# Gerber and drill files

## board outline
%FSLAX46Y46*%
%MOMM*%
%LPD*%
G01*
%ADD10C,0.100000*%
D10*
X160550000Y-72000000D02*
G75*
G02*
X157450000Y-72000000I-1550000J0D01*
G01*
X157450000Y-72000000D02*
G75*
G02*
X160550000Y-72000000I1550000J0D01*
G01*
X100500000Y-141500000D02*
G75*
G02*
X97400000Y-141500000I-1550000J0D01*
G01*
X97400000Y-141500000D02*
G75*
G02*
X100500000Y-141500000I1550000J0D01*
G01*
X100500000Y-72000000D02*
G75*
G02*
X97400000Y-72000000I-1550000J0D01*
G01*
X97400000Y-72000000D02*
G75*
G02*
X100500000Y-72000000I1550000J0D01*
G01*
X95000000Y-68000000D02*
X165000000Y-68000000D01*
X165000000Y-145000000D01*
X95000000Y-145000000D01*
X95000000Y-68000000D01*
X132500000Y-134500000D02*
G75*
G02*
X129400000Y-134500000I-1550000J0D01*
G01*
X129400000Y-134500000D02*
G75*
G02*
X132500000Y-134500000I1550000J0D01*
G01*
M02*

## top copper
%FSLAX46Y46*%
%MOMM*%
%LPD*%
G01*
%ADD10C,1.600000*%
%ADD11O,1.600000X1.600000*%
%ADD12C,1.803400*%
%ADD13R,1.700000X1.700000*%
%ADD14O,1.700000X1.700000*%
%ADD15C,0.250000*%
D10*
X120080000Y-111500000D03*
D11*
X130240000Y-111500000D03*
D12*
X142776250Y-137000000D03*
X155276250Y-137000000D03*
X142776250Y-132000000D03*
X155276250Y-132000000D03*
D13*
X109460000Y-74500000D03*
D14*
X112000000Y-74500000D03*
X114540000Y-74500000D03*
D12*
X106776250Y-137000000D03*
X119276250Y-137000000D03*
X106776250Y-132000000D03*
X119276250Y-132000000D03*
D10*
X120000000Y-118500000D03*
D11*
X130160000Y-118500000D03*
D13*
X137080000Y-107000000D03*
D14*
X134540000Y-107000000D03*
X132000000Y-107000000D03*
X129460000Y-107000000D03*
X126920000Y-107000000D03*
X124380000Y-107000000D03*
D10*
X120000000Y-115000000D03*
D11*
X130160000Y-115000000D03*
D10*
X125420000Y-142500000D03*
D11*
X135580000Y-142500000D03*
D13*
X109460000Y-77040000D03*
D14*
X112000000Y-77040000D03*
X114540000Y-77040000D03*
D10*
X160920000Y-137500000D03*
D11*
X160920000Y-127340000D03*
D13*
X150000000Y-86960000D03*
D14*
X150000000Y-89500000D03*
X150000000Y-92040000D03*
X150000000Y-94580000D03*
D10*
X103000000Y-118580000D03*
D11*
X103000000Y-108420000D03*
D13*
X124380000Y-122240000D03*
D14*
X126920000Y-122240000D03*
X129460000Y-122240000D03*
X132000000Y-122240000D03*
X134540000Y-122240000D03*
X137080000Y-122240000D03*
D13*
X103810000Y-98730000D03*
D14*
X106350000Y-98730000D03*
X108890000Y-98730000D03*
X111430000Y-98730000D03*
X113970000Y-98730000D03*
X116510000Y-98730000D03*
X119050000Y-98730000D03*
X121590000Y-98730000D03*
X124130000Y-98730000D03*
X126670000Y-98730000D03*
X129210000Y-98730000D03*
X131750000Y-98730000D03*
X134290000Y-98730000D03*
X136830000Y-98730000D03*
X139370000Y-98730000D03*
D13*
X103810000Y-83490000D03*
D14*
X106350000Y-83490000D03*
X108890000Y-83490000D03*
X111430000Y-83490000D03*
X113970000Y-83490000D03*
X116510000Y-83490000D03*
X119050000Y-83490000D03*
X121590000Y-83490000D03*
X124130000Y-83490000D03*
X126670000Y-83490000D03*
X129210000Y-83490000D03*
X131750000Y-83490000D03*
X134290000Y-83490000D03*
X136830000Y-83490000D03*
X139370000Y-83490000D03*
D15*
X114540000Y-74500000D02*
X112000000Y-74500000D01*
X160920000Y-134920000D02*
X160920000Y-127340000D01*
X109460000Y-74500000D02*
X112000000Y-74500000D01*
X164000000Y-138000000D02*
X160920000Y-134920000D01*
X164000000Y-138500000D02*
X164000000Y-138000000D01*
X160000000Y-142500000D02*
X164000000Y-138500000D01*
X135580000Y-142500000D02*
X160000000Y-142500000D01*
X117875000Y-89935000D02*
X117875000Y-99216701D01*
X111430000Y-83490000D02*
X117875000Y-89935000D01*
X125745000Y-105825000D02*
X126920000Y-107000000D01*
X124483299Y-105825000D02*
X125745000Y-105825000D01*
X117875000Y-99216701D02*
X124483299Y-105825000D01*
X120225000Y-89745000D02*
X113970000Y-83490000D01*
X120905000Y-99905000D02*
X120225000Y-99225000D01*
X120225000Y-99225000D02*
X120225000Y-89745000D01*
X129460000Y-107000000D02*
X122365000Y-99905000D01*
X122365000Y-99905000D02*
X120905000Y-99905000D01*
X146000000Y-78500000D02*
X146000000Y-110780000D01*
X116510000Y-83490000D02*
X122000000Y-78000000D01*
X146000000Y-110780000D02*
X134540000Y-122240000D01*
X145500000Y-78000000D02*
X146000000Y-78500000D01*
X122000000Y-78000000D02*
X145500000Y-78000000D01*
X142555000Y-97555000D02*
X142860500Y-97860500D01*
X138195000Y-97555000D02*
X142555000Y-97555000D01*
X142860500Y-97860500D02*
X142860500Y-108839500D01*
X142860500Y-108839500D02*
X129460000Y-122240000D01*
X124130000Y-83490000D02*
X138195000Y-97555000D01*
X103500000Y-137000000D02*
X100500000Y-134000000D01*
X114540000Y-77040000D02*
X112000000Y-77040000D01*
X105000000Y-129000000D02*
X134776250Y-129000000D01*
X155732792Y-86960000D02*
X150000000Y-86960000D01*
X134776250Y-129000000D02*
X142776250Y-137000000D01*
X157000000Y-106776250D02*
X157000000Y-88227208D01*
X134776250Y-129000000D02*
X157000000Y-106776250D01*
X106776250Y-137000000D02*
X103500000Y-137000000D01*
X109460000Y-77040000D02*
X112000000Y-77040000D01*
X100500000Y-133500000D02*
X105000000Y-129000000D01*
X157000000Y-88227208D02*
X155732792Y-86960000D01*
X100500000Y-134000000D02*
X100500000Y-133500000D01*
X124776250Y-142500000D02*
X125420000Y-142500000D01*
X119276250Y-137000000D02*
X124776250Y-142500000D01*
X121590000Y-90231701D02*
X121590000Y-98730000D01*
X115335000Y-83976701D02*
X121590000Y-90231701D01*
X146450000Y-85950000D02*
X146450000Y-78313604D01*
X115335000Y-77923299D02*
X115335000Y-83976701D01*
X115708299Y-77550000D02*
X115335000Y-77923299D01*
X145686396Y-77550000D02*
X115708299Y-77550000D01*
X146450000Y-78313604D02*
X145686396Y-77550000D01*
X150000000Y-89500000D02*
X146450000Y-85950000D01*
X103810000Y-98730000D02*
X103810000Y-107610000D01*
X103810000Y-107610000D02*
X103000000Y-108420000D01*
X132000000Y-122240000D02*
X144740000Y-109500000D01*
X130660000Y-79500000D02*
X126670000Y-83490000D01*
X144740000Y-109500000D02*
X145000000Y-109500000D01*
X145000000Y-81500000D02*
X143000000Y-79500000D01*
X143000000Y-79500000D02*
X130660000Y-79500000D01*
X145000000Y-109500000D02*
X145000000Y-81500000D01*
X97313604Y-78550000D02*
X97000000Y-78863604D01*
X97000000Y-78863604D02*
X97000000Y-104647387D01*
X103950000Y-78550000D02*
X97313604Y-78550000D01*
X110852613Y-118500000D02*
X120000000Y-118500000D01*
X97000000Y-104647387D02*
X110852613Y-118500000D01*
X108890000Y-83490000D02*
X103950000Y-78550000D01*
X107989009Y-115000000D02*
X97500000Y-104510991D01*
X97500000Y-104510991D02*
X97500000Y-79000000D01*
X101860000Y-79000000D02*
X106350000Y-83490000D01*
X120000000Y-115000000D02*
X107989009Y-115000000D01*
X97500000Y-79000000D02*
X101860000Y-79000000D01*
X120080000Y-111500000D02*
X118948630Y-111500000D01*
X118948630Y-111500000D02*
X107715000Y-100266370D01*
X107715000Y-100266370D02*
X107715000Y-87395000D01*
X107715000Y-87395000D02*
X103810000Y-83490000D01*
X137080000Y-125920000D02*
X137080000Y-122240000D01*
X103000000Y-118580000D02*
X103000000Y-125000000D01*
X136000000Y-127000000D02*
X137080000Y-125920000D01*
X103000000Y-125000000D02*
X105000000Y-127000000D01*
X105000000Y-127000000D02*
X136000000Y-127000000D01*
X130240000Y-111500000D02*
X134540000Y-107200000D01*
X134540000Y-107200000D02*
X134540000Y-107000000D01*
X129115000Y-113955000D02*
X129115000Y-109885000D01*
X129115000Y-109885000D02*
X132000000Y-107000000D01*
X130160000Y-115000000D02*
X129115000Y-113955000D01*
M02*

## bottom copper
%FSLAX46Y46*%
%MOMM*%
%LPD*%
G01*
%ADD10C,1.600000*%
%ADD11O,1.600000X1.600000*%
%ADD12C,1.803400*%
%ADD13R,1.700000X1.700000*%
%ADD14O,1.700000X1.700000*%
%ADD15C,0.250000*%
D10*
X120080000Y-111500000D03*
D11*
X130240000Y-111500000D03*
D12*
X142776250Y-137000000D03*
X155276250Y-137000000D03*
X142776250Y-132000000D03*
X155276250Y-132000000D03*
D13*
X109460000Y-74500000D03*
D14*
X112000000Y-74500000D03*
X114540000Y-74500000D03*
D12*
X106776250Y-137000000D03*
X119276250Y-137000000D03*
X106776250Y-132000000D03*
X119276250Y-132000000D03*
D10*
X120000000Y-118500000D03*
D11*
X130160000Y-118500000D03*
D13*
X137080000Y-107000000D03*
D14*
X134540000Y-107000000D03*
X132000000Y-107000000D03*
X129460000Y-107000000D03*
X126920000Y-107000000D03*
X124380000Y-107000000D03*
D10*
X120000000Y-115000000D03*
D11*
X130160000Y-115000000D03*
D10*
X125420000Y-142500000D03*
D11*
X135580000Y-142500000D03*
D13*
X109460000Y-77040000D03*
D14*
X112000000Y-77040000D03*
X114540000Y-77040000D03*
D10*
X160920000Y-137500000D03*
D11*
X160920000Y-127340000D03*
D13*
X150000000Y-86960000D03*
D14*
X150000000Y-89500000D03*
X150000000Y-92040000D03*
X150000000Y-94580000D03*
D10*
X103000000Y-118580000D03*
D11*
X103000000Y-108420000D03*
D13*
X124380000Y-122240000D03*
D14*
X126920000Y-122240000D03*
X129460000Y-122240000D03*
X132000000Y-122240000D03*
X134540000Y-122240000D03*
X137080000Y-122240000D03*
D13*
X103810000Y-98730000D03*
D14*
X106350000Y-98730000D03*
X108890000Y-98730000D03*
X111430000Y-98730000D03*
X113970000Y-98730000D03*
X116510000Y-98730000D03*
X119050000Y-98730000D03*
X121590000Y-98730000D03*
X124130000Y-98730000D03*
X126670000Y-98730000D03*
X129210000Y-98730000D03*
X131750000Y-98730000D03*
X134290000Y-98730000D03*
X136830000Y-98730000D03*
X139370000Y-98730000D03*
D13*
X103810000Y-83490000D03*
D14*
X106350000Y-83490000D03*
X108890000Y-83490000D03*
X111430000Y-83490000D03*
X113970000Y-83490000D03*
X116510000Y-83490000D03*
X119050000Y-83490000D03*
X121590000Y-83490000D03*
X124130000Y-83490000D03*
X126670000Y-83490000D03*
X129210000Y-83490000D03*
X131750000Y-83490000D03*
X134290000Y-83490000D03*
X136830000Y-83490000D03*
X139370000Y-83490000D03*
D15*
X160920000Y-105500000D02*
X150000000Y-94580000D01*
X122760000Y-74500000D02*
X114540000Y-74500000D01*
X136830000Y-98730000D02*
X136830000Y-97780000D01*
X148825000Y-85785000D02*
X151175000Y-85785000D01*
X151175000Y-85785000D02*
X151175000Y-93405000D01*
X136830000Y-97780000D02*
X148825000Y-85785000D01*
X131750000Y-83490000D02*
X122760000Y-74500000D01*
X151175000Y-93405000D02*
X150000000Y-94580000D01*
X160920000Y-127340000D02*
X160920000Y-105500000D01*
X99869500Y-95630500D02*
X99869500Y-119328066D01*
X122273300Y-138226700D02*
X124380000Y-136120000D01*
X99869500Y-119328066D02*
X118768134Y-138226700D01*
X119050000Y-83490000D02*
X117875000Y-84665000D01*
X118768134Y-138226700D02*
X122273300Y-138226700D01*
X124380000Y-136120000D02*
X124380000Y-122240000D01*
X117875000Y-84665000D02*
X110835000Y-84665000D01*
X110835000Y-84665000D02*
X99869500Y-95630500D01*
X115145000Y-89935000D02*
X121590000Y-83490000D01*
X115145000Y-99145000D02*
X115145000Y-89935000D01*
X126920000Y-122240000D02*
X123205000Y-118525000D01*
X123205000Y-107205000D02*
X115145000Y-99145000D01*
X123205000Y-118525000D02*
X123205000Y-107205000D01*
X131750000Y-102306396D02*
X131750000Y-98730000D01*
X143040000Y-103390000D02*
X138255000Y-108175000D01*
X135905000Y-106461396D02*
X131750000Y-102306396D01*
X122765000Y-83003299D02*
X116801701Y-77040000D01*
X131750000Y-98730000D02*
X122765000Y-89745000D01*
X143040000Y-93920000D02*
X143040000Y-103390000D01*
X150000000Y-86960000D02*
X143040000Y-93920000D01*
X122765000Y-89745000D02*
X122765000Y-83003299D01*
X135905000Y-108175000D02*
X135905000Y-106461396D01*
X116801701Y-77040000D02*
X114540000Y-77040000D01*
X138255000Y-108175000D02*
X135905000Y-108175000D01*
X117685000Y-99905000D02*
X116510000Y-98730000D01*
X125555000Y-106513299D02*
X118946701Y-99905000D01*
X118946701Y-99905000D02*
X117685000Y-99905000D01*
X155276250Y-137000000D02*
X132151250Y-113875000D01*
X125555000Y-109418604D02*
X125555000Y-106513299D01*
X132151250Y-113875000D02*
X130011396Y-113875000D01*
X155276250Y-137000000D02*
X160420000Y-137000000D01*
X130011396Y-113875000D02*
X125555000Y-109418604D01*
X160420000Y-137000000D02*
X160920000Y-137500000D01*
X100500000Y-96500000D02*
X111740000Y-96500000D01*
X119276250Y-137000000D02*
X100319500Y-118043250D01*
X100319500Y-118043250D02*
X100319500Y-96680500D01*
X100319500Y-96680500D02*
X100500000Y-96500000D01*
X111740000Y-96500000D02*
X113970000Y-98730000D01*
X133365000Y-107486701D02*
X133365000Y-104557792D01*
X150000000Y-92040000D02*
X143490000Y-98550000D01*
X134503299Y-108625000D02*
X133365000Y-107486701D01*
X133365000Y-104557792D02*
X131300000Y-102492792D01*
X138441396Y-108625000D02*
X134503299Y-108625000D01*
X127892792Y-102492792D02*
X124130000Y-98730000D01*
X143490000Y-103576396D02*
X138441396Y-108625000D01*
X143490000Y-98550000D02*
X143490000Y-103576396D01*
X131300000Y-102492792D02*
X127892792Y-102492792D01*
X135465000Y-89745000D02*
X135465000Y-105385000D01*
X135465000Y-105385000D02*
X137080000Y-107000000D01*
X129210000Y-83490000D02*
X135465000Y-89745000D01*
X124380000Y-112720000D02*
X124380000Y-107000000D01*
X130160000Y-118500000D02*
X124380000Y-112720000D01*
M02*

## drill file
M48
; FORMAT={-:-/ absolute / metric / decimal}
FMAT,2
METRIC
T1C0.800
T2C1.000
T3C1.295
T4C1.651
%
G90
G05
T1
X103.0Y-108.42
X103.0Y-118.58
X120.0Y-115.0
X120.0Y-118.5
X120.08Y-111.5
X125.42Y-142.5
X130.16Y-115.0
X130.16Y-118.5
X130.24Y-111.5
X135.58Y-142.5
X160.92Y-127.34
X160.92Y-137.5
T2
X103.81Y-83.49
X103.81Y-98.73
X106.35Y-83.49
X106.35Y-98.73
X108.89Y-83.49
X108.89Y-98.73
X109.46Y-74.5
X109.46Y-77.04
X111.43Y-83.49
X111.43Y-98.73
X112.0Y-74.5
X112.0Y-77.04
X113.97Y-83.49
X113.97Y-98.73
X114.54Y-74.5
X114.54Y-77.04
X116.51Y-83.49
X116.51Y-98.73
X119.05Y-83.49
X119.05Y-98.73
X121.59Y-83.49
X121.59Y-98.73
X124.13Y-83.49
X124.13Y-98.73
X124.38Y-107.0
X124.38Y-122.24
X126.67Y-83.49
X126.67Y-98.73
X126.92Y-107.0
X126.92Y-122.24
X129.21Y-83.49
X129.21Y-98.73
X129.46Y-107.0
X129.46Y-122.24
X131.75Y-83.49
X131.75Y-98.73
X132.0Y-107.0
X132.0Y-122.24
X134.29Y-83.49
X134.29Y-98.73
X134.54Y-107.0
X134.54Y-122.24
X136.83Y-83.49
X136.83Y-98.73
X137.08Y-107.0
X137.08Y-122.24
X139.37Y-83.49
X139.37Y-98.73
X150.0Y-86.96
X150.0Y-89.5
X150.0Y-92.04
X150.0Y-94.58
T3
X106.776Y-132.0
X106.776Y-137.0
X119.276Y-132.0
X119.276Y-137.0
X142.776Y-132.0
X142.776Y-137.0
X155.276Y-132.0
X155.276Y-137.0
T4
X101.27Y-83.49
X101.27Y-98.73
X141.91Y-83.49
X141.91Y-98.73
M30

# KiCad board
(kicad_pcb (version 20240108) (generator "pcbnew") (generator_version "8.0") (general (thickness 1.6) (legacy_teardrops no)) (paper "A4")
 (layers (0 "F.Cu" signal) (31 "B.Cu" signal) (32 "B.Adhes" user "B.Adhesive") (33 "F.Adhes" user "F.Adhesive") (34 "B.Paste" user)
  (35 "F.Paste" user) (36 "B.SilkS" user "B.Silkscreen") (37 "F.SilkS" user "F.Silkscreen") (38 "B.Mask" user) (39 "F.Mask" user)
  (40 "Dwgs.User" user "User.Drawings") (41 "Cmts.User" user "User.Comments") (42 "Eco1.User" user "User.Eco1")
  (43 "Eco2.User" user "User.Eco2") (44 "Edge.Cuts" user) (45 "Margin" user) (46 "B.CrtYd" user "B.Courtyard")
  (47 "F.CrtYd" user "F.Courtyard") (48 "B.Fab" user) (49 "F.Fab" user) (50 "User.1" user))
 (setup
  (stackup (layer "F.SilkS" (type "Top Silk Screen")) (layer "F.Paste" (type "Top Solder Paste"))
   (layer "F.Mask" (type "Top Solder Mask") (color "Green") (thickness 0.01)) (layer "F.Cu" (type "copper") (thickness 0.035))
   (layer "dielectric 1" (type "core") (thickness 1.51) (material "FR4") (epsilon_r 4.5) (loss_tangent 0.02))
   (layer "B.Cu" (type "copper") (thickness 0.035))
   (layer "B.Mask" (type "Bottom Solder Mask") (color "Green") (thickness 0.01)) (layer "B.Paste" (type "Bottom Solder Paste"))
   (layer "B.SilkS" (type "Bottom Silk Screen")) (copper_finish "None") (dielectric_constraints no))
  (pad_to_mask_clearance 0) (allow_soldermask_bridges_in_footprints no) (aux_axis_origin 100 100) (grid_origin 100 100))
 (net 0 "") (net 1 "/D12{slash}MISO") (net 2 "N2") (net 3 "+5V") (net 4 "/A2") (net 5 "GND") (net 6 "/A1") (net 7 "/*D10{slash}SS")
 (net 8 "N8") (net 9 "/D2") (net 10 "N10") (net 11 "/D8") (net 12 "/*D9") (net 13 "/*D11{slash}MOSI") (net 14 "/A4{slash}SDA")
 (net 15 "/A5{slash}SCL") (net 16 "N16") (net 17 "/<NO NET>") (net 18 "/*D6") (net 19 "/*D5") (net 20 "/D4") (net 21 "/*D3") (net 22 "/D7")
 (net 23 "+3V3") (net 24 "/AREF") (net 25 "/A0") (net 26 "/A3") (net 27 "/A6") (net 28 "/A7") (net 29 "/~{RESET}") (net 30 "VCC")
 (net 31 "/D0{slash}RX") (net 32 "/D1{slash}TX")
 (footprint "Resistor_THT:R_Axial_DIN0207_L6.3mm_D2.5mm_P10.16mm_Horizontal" (layer "F.Cu") (at 120.08 111.5)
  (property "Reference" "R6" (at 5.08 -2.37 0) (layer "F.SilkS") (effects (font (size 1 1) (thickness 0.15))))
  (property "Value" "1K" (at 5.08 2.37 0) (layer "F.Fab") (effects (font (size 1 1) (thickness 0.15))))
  (pad "1" thru_hole circle (at 0 0) (size 1.6 1.6) (drill 0.8) (layers "*.Cu" "*.Mask") (remove_unused_layers no) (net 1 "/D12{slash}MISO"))
  (pad "2" thru_hole oval (at 10.16 0) (size 1.6 1.6) (drill 0.8) (layers "*.Cu" "*.Mask") (remove_unused_layers no) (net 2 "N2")))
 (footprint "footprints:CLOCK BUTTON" (layer "F.Cu") (at 142.77625 137)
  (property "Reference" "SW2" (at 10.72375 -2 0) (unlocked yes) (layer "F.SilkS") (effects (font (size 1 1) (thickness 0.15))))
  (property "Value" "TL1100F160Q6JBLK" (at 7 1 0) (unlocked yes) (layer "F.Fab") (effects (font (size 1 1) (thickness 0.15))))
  (pad "1" thru_hole circle (at 0 0) (size 1.8034 1.8034) (drill 1.2954) (layers "*.Cu" "*.Mask") (remove_unused_layers no) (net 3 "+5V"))
  (pad "2" thru_hole circle (at 12.5 0) (size 1.8034 1.8034) (drill 1.2954) (layers "*.Cu" "*.Mask") (remove_unused_layers no) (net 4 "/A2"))
  (pad "3" thru_hole circle (at 0 -5) (size 1.8034 1.8034) (drill 1.2954) (layers "*.Cu" "*.Mask") (remove_unused_layers no))
  (pad "4" thru_hole circle (at 12.5 -5) (size 1.8034 1.8034) (drill 1.2954) (layers "*.Cu" "*.Mask") (remove_unused_layers no)))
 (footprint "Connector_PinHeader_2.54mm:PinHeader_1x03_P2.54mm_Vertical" (layer "F.Cu") (at 109.46 74.5 90)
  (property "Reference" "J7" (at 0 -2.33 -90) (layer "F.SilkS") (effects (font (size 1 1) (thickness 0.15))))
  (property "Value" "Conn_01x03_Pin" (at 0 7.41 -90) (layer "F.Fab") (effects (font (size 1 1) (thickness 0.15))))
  (pad "1" thru_hole rect (at 0 0 90) (size 1.7 1.7) (drill 1) (layers "*.Cu" "*.Mask") (remove_unused_layers no) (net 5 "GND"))
  (pad "2" thru_hole oval (at 0 2.54 90) (size 1.7 1.7) (drill 1) (layers "*.Cu" "*.Mask") (remove_unused_layers no) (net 5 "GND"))
  (pad "3" thru_hole oval (at 0 5.08 90) (size 1.7 1.7) (drill 1) (layers "*.Cu" "*.Mask") (remove_unused_layers no) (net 5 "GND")))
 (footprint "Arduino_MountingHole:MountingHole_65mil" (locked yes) (layer "F.Cu") (at 101.27 83.49)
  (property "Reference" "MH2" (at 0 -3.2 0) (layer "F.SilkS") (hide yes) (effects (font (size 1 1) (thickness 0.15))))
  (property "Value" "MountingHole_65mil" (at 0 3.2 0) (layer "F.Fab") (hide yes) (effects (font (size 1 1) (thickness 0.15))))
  (pad "" np_thru_hole circle (at 0 0) (size 1.651 1.651) (drill 1.651) (layers "F&B.Cu" "*.Mask")))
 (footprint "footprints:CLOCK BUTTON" (layer "F.Cu") (at 106.77625 137)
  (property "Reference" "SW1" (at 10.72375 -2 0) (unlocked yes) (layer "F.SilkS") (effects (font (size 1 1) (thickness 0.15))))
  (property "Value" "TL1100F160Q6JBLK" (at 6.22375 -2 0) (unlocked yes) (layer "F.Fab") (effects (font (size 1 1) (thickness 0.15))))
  (pad "1" thru_hole circle (at 0 0) (size 1.8034 1.8034) (drill 1.2954) (layers "*.Cu" "*.Mask") (remove_unused_layers no) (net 3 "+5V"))
  (pad "2" thru_hole circle (at 12.5 0) (size 1.8034 1.8034) (drill 1.2954) (layers "*.Cu" "*.Mask") (remove_unused_layers no) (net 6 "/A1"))
  (pad "3" thru_hole circle (at 0 -5) (size 1.8034 1.8034) (drill 1.2954) (layers "*.Cu" "*.Mask") (remove_unused_layers no))
  (pad "4" thru_hole circle (at 12.5 -5) (size 1.8034 1.8034) (drill 1.2954) (layers "*.Cu" "*.Mask") (remove_unused_layers no)))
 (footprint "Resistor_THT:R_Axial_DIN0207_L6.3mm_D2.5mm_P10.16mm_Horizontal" (layer "F.Cu") (at 120 118.5)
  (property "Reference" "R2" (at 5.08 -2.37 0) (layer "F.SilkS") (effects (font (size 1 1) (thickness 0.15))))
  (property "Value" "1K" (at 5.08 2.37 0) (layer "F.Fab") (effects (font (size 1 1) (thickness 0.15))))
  (pad "1" thru_hole circle (at 0 0) (size 1.6 1.6) (drill 0.8) (layers "*.Cu" "*.Mask") (remove_unused_layers no) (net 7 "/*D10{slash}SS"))
  (pad "2" thru_hole oval (at 10.16 0) (size 1.6 1.6) (drill 0.8) (layers "*.Cu" "*.Mask") (remove_unused_layers no) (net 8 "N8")))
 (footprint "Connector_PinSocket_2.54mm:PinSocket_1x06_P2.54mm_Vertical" (layer "F.Cu") (at 137.08 107 -90)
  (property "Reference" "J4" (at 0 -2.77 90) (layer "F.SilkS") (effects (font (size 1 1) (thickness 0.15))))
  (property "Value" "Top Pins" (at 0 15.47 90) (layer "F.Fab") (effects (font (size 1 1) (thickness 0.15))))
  (pad "1" thru_hole rect (at 0 0 270) (size 1.7 1.7) (drill 1) (layers "*.Cu" "*.Mask") (remove_unused_layers no) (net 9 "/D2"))
  (pad "2" thru_hole oval (at 0 2.54 270) (size 1.7 1.7) (drill 1) (layers "*.Cu" "*.Mask") (remove_unused_layers no) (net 2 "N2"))
  (pad "3" thru_hole oval (at 0 5.08 270) (size 1.7 1.7) (drill 1) (layers "*.Cu" "*.Mask") (remove_unused_layers no) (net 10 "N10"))
  (pad "4" thru_hole oval (at 0 7.62 270) (size 1.7 1.7) (drill 1) (layers "*.Cu" "*.Mask") (remove_unused_layers no) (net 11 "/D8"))
  (pad "5" thru_hole oval (at 0 10.16 270) (size 1.7 1.7) (drill 1) (layers "*.Cu" "*.Mask") (remove_unused_layers no) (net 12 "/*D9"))
  (pad "6" thru_hole oval (at 0 12.7 270) (size 1.7 1.7) (drill 1) (layers "*.Cu" "*.Mask") (remove_unused_layers no) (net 8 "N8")))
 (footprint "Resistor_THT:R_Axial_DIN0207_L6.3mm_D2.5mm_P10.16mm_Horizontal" (layer "F.Cu") (at 120 115)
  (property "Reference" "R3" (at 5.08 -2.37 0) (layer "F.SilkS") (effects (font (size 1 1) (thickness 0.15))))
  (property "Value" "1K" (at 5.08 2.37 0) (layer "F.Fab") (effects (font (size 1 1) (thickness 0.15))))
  (pad "1" thru_hole circle (at 0 0) (size 1.6 1.6) (drill 0.8) (layers "*.Cu" "*.Mask") (remove_unused_layers no)
   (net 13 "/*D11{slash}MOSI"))
  (pad "2" thru_hole oval (at 10.16 0) (size 1.6 1.6) (drill 0.8) (layers "*.Cu" "*.Mask") (remove_unused_layers no) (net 10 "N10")))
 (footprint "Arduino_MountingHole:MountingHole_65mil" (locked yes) (layer "F.Cu") (at 141.91 98.73)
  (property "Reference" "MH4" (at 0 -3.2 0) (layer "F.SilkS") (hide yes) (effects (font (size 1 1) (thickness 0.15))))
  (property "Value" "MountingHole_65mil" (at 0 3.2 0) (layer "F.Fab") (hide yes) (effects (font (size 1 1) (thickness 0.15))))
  (pad "" np_thru_hole circle (at 0 0) (size 1.651 1.651) (drill 1.651) (layers "F&B.Cu" "*.Mask")))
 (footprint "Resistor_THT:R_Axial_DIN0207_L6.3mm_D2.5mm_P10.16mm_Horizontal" (layer "F.Cu") (at 125.42 142.5)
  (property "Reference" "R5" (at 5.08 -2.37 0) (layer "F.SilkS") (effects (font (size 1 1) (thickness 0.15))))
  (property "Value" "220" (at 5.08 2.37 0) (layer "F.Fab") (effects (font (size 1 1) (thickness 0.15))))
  (pad "1" thru_hole circle (at 0 0) (size 1.6 1.6) (drill 0.8) (layers "*.Cu" "*.Mask") (remove_unused_layers no) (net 6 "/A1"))
  (pad "2" thru_hole oval (at 10.16 0) (size 1.6 1.6) (drill 0.8) (layers "*.Cu" "*.Mask") (remove_unused_layers no) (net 5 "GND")))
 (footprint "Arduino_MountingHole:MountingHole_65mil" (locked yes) (layer "F.Cu") (at 101.27 98.73)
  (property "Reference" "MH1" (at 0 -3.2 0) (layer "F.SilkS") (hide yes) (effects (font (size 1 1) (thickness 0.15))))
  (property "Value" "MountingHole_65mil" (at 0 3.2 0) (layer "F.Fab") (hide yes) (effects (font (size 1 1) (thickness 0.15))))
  (pad "" np_thru_hole circle (at 0 0) (size 1.651 1.651) (drill 1.651) (layers "F&B.Cu" "*.Mask")))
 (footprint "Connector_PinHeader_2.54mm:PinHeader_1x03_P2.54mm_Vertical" (layer "F.Cu") (at 109.46 77.04 90)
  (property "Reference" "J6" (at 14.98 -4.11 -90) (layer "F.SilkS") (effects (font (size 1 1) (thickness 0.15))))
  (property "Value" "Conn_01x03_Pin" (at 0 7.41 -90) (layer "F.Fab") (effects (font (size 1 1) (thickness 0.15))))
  (pad "1" thru_hole rect (at 0 0 90) (size 1.7 1.7) (drill 1) (layers "*.Cu" "*.Mask") (remove_unused_layers no) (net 3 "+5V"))
  (pad "2" thru_hole oval (at 0 2.54 90) (size 1.7 1.7) (drill 1) (layers "*.Cu" "*.Mask") (remove_unused_layers no) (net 3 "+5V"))
  (pad "3" thru_hole oval (at 0 5.08 90) (size 1.7 1.7) (drill 1) (layers "*.Cu" "*.Mask") (remove_unused_layers no) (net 3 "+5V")))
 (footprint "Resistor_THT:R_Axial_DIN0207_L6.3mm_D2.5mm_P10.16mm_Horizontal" (layer "F.Cu") (at 160.92 137.5 90)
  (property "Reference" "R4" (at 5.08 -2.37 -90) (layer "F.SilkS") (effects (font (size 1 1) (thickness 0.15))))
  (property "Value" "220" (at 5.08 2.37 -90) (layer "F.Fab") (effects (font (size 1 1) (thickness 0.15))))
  (pad "1" thru_hole circle (at 0 0 90) (size 1.6 1.6) (drill 0.8) (layers "*.Cu" "*.Mask") (remove_unused_layers no) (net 4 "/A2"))
  (pad "2" thru_hole oval (at 10.16 0 90) (size 1.6 1.6) (drill 0.8) (layers "*.Cu" "*.Mask") (remove_unused_layers no) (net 5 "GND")))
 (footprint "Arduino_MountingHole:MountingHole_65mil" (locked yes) (layer "F.Cu") (at 141.91 83.49)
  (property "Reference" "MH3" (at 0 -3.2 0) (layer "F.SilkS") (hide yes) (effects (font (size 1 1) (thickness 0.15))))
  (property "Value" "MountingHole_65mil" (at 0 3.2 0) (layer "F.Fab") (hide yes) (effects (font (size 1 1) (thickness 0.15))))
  (pad "" np_thru_hole circle (at 0 0) (size 1.651 1.651) (drill 1.651) (layers "F&B.Cu" "*.Mask")))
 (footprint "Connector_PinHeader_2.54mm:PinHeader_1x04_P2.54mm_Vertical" (layer "F.Cu") (at 150 86.96)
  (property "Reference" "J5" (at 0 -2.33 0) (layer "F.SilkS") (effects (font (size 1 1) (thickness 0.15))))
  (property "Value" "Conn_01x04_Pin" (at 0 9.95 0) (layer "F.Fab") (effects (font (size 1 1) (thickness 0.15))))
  (pad "1" thru_hole rect (at 0 0) (size 1.7 1.7) (drill 1) (layers "*.Cu" "*.Mask") (remove_unused_layers no) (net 3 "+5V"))
  (pad "2" thru_hole oval (at 0 2.54) (size 1.7 1.7) (drill 1) (layers "*.Cu" "*.Mask") (remove_unused_layers no) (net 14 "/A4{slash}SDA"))
  (pad "3" thru_hole oval (at 0 5.08) (size 1.7 1.7) (drill 1) (layers "*.Cu" "*.Mask") (remove_unused_layers no) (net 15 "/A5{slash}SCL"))
  (pad "4" thru_hole oval (at 0 7.62) (size 1.7 1.7) (drill 1) (layers "*.Cu" "*.Mask") (remove_unused_layers no) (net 5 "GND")))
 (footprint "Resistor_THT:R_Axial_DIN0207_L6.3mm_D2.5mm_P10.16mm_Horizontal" (layer "F.Cu") (at 103 118.58 90)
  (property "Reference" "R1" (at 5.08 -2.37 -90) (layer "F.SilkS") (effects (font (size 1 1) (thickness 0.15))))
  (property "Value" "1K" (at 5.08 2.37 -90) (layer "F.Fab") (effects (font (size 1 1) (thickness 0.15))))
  (pad "1" thru_hole circle (at 0 0 90) (size 1.6 1.6) (drill 0.8) (layers "*.Cu" "*.Mask") (remove_unused_layers no) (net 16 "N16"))
  (pad "2" thru_hole oval (at 10.16 0 90) (size 1.6 1.6) (drill 0.8) (layers "*.Cu" "*.Mask") (remove_unused_layers no) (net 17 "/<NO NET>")))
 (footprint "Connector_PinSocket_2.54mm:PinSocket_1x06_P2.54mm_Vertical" (layer "F.Cu") (at 124.38 122.24 90)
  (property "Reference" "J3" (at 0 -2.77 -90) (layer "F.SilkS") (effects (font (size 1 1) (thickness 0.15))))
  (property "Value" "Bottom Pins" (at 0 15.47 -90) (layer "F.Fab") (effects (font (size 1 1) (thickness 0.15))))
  (pad "1" thru_hole rect (at 0 0 90) (size 1.7 1.7) (drill 1) (layers "*.Cu" "*.Mask") (remove_unused_layers no) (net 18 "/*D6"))
  (pad "2" thru_hole oval (at 0 2.54 90) (size 1.7 1.7) (drill 1) (layers "*.Cu" "*.Mask") (remove_unused_layers no) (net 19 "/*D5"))
  (pad "3" thru_hole oval (at 0 5.08 90) (size 1.7 1.7) (drill 1) (layers "*.Cu" "*.Mask") (remove_unused_layers no) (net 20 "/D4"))
  (pad "4" thru_hole oval (at 0 7.62 90) (size 1.7 1.7) (drill 1) (layers "*.Cu" "*.Mask") (remove_unused_layers no) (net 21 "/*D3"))
  (pad "5" thru_hole oval (at 0 10.16 90) (size 1.7 1.7) (drill 1) (layers "*.Cu" "*.Mask") (remove_unused_layers no) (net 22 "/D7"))
  (pad "6" thru_hole oval (at 0 12.7 90) (size 1.7 1.7) (drill 1) (layers "*.Cu" "*.Mask") (remove_unused_layers no) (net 16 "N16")))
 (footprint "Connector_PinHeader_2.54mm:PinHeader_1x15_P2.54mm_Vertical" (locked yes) (layer "B.Cu") (at 103.81 98.73 -90)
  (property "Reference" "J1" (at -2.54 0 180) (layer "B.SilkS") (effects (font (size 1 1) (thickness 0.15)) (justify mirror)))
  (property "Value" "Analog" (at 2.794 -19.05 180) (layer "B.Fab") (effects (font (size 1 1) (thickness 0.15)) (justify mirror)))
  (pad "1" thru_hole rect (at 0 0 270) (size 1.7 1.7) (drill 1) (layers "*.Cu" "*.Mask") (remove_unused_layers no) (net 17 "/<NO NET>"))
  (pad "2" thru_hole oval (at 0 -2.54 270) (size 1.7 1.7) (drill 1) (layers "*.Cu" "*.Mask") (remove_unused_layers no) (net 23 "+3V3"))
  (pad "3" thru_hole oval (at 0 -5.08 270) (size 1.7 1.7) (drill 1) (layers "*.Cu" "*.Mask") (remove_unused_layers no) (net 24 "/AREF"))
  (pad "4" thru_hole oval (at 0 -7.62 270) (size 1.7 1.7) (drill 1) (layers "*.Cu" "*.Mask") (remove_unused_layers no) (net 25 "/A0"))
  (pad "5" thru_hole oval (at 0 -10.16 270) (size 1.7 1.7) (drill 1) (layers "*.Cu" "*.Mask") (remove_unused_layers no) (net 6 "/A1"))
  (pad "6" thru_hole oval (at 0 -12.7 270) (size 1.7 1.7) (drill 1) (layers "*.Cu" "*.Mask") (remove_unused_layers no) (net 4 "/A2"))
  (pad "7" thru_hole oval (at 0 -15.24 270) (size 1.7 1.7) (drill 1) (layers "*.Cu" "*.Mask") (remove_unused_layers no) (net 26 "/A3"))
  (pad "8" thru_hole oval (at 0 -17.78 270) (size 1.7 1.7) (drill 1) (layers "*.Cu" "*.Mask") (remove_unused_layers no)
   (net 14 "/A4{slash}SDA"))
  (pad "9" thru_hole oval (at 0 -20.32 270) (size 1.7 1.7) (drill 1) (layers "*.Cu" "*.Mask") (remove_unused_layers no)
   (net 15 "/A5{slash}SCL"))
  (pad "10" thru_hole oval (at 0 -22.86 270) (size 1.7 1.7) (drill 1) (layers "*.Cu" "*.Mask") (remove_unused_layers no) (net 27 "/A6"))
  (pad "11" thru_hole oval (at 0 -25.4 270) (size 1.7 1.7) (drill 1) (layers "*.Cu" "*.Mask") (remove_unused_layers no) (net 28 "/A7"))
  (pad "12" thru_hole oval (at 0 -27.94 270) (size 1.7 1.7) (drill 1) (layers "*.Cu" "*.Mask") (remove_unused_layers no) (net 3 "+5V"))
  (pad "13" thru_hole oval (at 0 -30.48 270) (size 1.7 1.7) (drill 1) (layers "*.Cu" "*.Mask") (remove_unused_layers no)
   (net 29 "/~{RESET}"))
  (pad "14" thru_hole oval (at 0 -33.02 270) (size 1.7 1.7) (drill 1) (layers "*.Cu" "*.Mask") (remove_unused_layers no) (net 5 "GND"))
  (pad "15" thru_hole oval (at 0 -35.56 270) (size 1.7 1.7) (drill 1) (layers "*.Cu" "*.Mask") (remove_unused_layers no) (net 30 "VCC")))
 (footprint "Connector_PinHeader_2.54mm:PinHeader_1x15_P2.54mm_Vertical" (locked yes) (layer "B.Cu") (at 103.81 83.49 -90)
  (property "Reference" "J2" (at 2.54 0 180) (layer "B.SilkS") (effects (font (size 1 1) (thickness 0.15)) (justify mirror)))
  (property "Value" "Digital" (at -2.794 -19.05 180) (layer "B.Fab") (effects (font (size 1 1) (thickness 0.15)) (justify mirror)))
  (pad "1" thru_hole rect (at 0 0 270) (size 1.7 1.7) (drill 1) (layers "*.Cu" "*.Mask") (remove_unused_layers no) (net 1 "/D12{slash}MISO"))
  (pad "2" thru_hole oval (at 0 -2.54 270) (size 1.7 1.7) (drill 1) (layers "*.Cu" "*.Mask") (remove_unused_layers no)
   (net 13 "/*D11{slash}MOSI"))
  (pad "3" thru_hole oval (at 0 -5.08 270) (size 1.7 1.7) (drill 1) (layers "*.Cu" "*.Mask") (remove_unused_layers no)
   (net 7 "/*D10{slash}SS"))
  (pad "4" thru_hole oval (at 0 -7.62 270) (size 1.7 1.7) (drill 1) (layers "*.Cu" "*.Mask") (remove_unused_layers no) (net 12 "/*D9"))
  (pad "5" thru_hole oval (at 0 -10.16 270) (size 1.7 1.7) (drill 1) (layers "*.Cu" "*.Mask") (remove_unused_layers no) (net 11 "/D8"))
  (pad "6" thru_hole oval (at 0 -12.7 270) (size 1.7 1.7) (drill 1) (layers "*.Cu" "*.Mask") (remove_unused_layers no) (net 22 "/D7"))
  (pad "7" thru_hole oval (at 0 -15.24 270) (size 1.7 1.7) (drill 1) (layers "*.Cu" "*.Mask") (remove_unused_layers no) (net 18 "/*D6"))
  (pad "8" thru_hole oval (at 0 -17.78 270) (size 1.7 1.7) (drill 1) (layers "*.Cu" "*.Mask") (remove_unused_layers no) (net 19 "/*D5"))
  (pad "9" thru_hole oval (at 0 -20.32 270) (size 1.7 1.7) (drill 1) (layers "*.Cu" "*.Mask") (remove_unused_layers no) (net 20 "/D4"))
  (pad "10" thru_hole oval (at 0 -22.86 270) (size 1.7 1.7) (drill 1) (layers "*.Cu" "*.Mask") (remove_unused_layers no) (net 21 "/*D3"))
  (pad "11" thru_hole oval (at 0 -25.4 270) (size 1.7 1.7) (drill 1) (layers "*.Cu" "*.Mask") (remove_unused_layers no) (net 9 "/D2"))
  (pad "12" thru_hole oval (at 0 -27.94 270) (size 1.7 1.7) (drill 1) (layers "*.Cu" "*.Mask") (remove_unused_layers no) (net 5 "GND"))
  (pad "13" thru_hole oval (at 0 -30.48 270) (size 1.7 1.7) (drill 1) (layers "*.Cu" "*.Mask") (remove_unused_layers no)
   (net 29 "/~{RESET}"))
  (pad "14" thru_hole oval (at 0 -33.02 270) (size 1.7 1.7) (drill 1) (layers "*.Cu" "*.Mask") (remove_unused_layers no)
   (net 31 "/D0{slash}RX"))
  (pad "15" thru_hole oval (at 0 -35.56 270) (size 1.7 1.7) (drill 1) (layers "*.Cu" "*.Mask") (remove_unused_layers no)
   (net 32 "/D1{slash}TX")))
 (gr_circle (center 159 72) (end 160.55 72) (stroke (width 0.1) (type default)) (fill none) (layer "Edge.Cuts"))
 (gr_circle (center 98.95 141.5) (end 100.5 141.5) (stroke (width 0.1) (type default)) (fill none) (layer "Edge.Cuts"))
 (gr_circle (center 98.95 72) (end 100.5 72) (stroke (width 0.1) (type default)) (fill none) (layer "Edge.Cuts"))
 (gr_rect (start 95 68) (end 165 145) (stroke (width 0.1) (type default)) (fill none) (layer "Edge.Cuts"))
 (gr_circle (center 130.95 134.5) (end 132.5 134.5) (stroke (width 0.1) (type default)) (fill none) (layer "Edge.Cuts"))
 (segment (start 114.54 74.5) (end 112 74.5) (width 0.25) (layer "F.Cu") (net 5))
 (segment (start 160.92 134.92) (end 160.92 127.34) (width 0.25) (layer "F.Cu") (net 5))
 (segment (start 109.46 74.5) (end 112 74.5) (width 0.25) (layer "F.Cu") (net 5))
 (segment (start 164 138) (end 160.92 134.92) (width 0.25) (layer "F.Cu") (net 5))
 (segment (start 164 138.5) (end 164 138) (width 0.25) (layer "F.Cu") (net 5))
 (segment (start 160 142.5) (end 164 138.5) (width 0.25) (layer "F.Cu") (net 5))
 (segment (start 135.58 142.5) (end 160 142.5) (width 0.25) (layer "F.Cu") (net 5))
 (segment (start 160.92 105.5) (end 150 94.58) (width 0.25) (layer "B.Cu") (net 5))
 (segment (start 122.76 74.5) (end 114.54 74.5) (width 0.25) (layer "B.Cu") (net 5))
 (segment (start 136.83 98.73) (end 136.83 97.78) (width 0.25) (layer "B.Cu") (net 5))
 (segment (start 148.825 85.785) (end 151.175 85.785) (width 0.25) (layer "B.Cu") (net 5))
 (segment (start 151.175 85.785) (end 151.175 93.405) (width 0.25) (layer "B.Cu") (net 5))
 (segment (start 136.83 97.78) (end 148.825 85.785) (width 0.25) (layer "B.Cu") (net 5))
 (segment (start 131.75 83.49) (end 122.76 74.5) (width 0.25) (layer "B.Cu") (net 5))
 (segment (start 151.175 93.405) (end 150 94.58) (width 0.25) (layer "B.Cu") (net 5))
 (segment (start 160.92 127.34) (end 160.92 105.5) (width 0.25) (layer "B.Cu") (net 5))
 (segment (start 117.875 89.935) (end 117.875 99.216701) (width 0.25) (layer "F.Cu") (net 12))
 (segment (start 111.43 83.49) (end 117.875 89.935) (width 0.25) (layer "F.Cu") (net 12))
 (segment (start 125.745 105.825) (end 126.92 107) (width 0.25) (layer "F.Cu") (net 12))
 (segment (start 124.483299 105.825) (end 125.745 105.825) (width 0.25) (layer "F.Cu") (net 12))
 (segment (start 117.875 99.216701) (end 124.483299 105.825) (width 0.25) (layer "F.Cu") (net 12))
 (segment (start 120.225 89.745) (end 113.97 83.49) (width 0.25) (layer "F.Cu") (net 11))
 (segment (start 120.905 99.905) (end 120.225 99.225) (width 0.25) (layer "F.Cu") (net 11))
 (segment (start 120.225 99.225) (end 120.225 89.745) (width 0.25) (layer "F.Cu") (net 11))
 (segment (start 129.46 107) (end 122.365 99.905) (width 0.25) (layer "F.Cu") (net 11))
 (segment (start 122.365 99.905) (end 120.905 99.905) (width 0.25) (layer "F.Cu") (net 11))
 (segment (start 146 78.5) (end 146 110.78) (width 0.25) (layer "F.Cu") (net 22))
 (segment (start 116.51 83.49) (end 122 78) (width 0.25) (layer "F.Cu") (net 22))
 (segment (start 146 110.78) (end 134.54 122.24) (width 0.25) (layer "F.Cu") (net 22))
 (segment (start 145.5 78) (end 146 78.5) (width 0.25) (layer "F.Cu") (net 22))
 (segment (start 122 78) (end 145.5 78) (width 0.25) (layer "F.Cu") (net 22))
 (segment (start 99.8695 95.6305) (end 99.8695 119.328066) (width 0.25) (layer "B.Cu") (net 18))
 (segment (start 122.2733 138.2267) (end 124.38 136.12) (width 0.25) (layer "B.Cu") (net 18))
 (segment (start 99.8695 119.328066) (end 118.768134 138.2267) (width 0.25) (layer "B.Cu") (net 18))
 (segment (start 119.05 83.49) (end 117.875 84.665) (width 0.25) (layer "B.Cu") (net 18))
 (segment (start 118.768134 138.2267) (end 122.2733 138.2267) (width 0.25) (layer "B.Cu") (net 18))
 (segment (start 124.38 136.12) (end 124.38 122.24) (width 0.25) (layer "B.Cu") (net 18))
 (segment (start 117.875 84.665) (end 110.835 84.665) (width 0.25) (layer "B.Cu") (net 18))
 (segment (start 110.835 84.665) (end 99.8695 95.6305) (width 0.25) (layer "B.Cu") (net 18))
 (segment (start 115.145 89.935) (end 121.59 83.49) (width 0.25) (layer "B.Cu") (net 19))
 (segment (start 115.145 99.145) (end 115.145 89.935) (width 0.25) (layer "B.Cu") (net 19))
 (segment (start 126.92 122.24) (end 123.205 118.525) (width 0.25) (layer "B.Cu") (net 19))
 (segment (start 123.205 107.205) (end 115.145 99.145) (width 0.25) (layer "B.Cu") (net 19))
 (segment (start 123.205 118.525) (end 123.205 107.205) (width 0.25) (layer "B.Cu") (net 19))
 (segment (start 142.555 97.555) (end 142.8605 97.8605) (width 0.25) (layer "F.Cu") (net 20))
 (segment (start 138.195 97.555) (end 142.555 97.555) (width 0.25) (layer "F.Cu") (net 20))
 (segment (start 142.8605 97.8605) (end 142.8605 108.8395) (width 0.25) (layer "F.Cu") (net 20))
 (segment (start 142.8605 108.8395) (end 129.46 122.24) (width 0.25) (layer "F.Cu") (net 20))
 (segment (start 124.13 83.49) (end 138.195 97.555) (width 0.25) (layer "F.Cu") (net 20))
 (segment (start 103.5 137) (end 100.5 134) (width 0.25) (layer "F.Cu") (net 3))
 (segment (start 114.54 77.04) (end 112 77.04) (width 0.25) (layer "F.Cu") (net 3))
 (segment (start 105 129) (end 134.77625 129) (width 0.25) (layer "F.Cu") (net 3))
 (segment (start 155.732792 86.96) (end 150 86.96) (width 0.25) (layer "F.Cu") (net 3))
 (segment (start 134.77625 129) (end 142.77625 137) (width 0.25) (layer "F.Cu") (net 3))
 (segment (start 157 106.77625) (end 157 88.227208) (width 0.25) (layer "F.Cu") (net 3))
 (segment (start 134.77625 129) (end 157 106.77625) (width 0.25) (layer "F.Cu") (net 3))
 (segment (start 106.77625 137) (end 103.5 137) (width 0.25) (layer "F.Cu") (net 3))
 (segment (start 109.46 77.04) (end 112 77.04) (width 0.25) (layer "F.Cu") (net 3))
 (segment (start 100.5 133.5) (end 105 129) (width 0.25) (layer "F.Cu") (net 3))
 (segment (start 157 88.227208) (end 155.732792 86.96) (width 0.25) (layer "F.Cu") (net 3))
 (segment (start 100.5 134) (end 100.5 133.5) (width 0.25) (layer "F.Cu") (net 3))
 (segment (start 131.75 102.306396) (end 131.75 98.73) (width 0.25) (layer "B.Cu") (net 3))
 (segment (start 143.04 103.39) (end 138.255 108.175) (width 0.25) (layer "B.Cu") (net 3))
 (segment (start 135.905 106.461396) (end 131.75 102.306396) (width 0.25) (layer "B.Cu") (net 3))
 (segment (start 122.765 83.003299) (end 116.801701 77.04) (width 0.25) (layer "B.Cu") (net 3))
 (segment (start 131.75 98.73) (end 122.765 89.745) (width 0.25) (layer "B.Cu") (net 3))
 (segment (start 143.04 93.92) (end 143.04 103.39) (width 0.25) (layer "B.Cu") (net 3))
 (segment (start 150 86.96) (end 143.04 93.92) (width 0.25) (layer "B.Cu") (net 3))
 (segment (start 122.765 89.745) (end 122.765 83.003299) (width 0.25) (layer "B.Cu") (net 3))
 (segment (start 135.905 108.175) (end 135.905 106.461396) (width 0.25) (layer "B.Cu") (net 3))
 (segment (start 116.801701 77.04) (end 114.54 77.04) (width 0.25) (layer "B.Cu") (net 3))
 (segment (start 138.255 108.175) (end 135.905 108.175) (width 0.25) (layer "B.Cu") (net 3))
 (segment (start 117.685 99.905) (end 116.51 98.73) (width 0.25) (layer "B.Cu") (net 4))
 (segment (start 125.555 106.513299) (end 118.946701 99.905) (width 0.25) (layer "B.Cu") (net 4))
 (segment (start 118.946701 99.905) (end 117.685 99.905) (width 0.25) (layer "B.Cu") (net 4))
 (segment (start 155.27625 137) (end 132.15125 113.875) (width 0.25) (layer "B.Cu") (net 4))
 (segment (start 125.555 109.418604) (end 125.555 106.513299) (width 0.25) (layer "B.Cu") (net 4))
 (segment (start 132.15125 113.875) (end 130.011396 113.875) (width 0.25) (layer "B.Cu") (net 4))
 (segment (start 155.27625 137) (end 160.42 137) (width 0.25) (layer "B.Cu") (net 4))
 (segment (start 130.011396 113.875) (end 125.555 109.418604) (width 0.25) (layer "B.Cu") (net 4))
 (segment (start 160.42 137) (end 160.92 137.5) (width 0.25) (layer "B.Cu") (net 4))
 (segment (start 124.77625 142.5) (end 125.42 142.5) (width 0.25) (layer "F.Cu") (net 6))
 (segment (start 119.27625 137) (end 124.77625 142.5) (width 0.25) (layer "F.Cu") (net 6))
 (segment (start 100.5 96.5) (end 111.74 96.5) (width 0.25) (layer "B.Cu") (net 6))
 (segment (start 119.27625 137) (end 100.3195 118.04325) (width 0.25) (layer "B.Cu") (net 6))
 (segment (start 100.3195 118.04325) (end 100.3195 96.6805) (width 0.25) (layer "B.Cu") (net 6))
 (segment (start 100.3195 96.6805) (end 100.5 96.5) (width 0.25) (layer "B.Cu") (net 6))
 (segment (start 111.74 96.5) (end 113.97 98.73) (width 0.25) (layer "B.Cu") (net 6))
 (segment (start 133.365 107.486701) (end 133.365 104.557792) (width 0.25) (layer "B.Cu") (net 15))
 (segment (start 150 92.04) (end 143.49 98.55) (width 0.25) (layer "B.Cu") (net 15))
 (segment (start 134.503299 108.625) (end 133.365 107.486701) (width 0.25) (layer "B.Cu") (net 15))
 (segment (start 133.365 104.557792) (end 131.3 102.492792) (width 0.25) (layer "B.Cu") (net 15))
 (segment (start 138.441396 108.625) (end 134.503299 108.625) (width 0.25) (layer "B.Cu") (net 15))
 (segment (start 127.892792 102.492792) (end 124.13 98.73) (width 0.25) (layer "B.Cu") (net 15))
 (segment (start 143.49 103.576396) (end 138.441396 108.625) (width 0.25) (layer "B.Cu") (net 15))
 (segment (start 143.49 98.55) (end 143.49 103.576396) (width 0.25) (layer "B.Cu") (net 15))
 (segment (start 131.3 102.492792) (end 127.892792 102.492792) (width 0.25) (layer "B.Cu") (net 15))
 (segment (start 121.59 90.231701) (end 121.59 98.73) (width 0.25) (layer "F.Cu") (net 14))
 (segment (start 115.335 83.976701) (end 121.59 90.231701) (width 0.25) (layer "F.Cu") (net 14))
 (segment (start 146.45 85.95) (end 146.45 78.313604) (width 0.25) (layer "F.Cu") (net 14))
 (segment (start 115.335 77.923299) (end 115.335 83.976701) (width 0.25) (layer "F.Cu") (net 14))
 (segment (start 115.708299 77.55) (end 115.335 77.923299) (width 0.25) (layer "F.Cu") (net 14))
 (segment (start 145.686396 77.55) (end 115.708299 77.55) (width 0.25) (layer "F.Cu") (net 14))
 (segment (start 146.45 78.313604) (end 145.686396 77.55) (width 0.25) (layer "F.Cu") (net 14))
 (segment (start 150 89.5) (end 146.45 85.95) (width 0.25) (layer "F.Cu") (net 14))
 (segment (start 103.81 98.73) (end 103.81 107.61) (width 0.25) (layer "F.Cu") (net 17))
 (segment (start 103.81 107.61) (end 103 108.42) (width 0.25) (layer "F.Cu") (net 17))
 (segment (start 135.465 89.745) (end 135.465 105.385) (width 0.25) (layer "B.Cu") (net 9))
 (segment (start 135.465 105.385) (end 137.08 107) (width 0.25) (layer "B.Cu") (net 9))
 (segment (start 129.21 83.49) (end 135.465 89.745) (width 0.25) (layer "B.Cu") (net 9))
 (segment (start 132 122.24) (end 144.74 109.5) (width 0.25) (layer "F.Cu") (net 21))
 (segment (start 130.66 79.5) (end 126.67 83.49) (width 0.25) (layer "F.Cu") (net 21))
 (segment (start 144.74 109.5) (end 145 109.5) (width 0.25) (layer "F.Cu") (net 21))
 (segment (start 145 81.5) (end 143 79.5) (width 0.25) (layer "F.Cu") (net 21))
 (segment (start 143 79.5) (end 130.66 79.5) (width 0.25) (layer "F.Cu") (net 21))
 (segment (start 145 109.5) (end 145 81.5) (width 0.25) (layer "F.Cu") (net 21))
 (segment (start 97.313604 78.55) (end 97 78.863604) (width 0.25) (layer "F.Cu") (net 7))
 (segment (start 97 78.863604) (end 97 104.647387) (width 0.25) (layer "F.Cu") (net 7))
 (segment (start 103.95 78.55) (end 97.313604 78.55) (width 0.25) (layer "F.Cu") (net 7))
 (segment (start 110.852613 118.5) (end 120 118.5) (width 0.25) (layer "F.Cu") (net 7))
 (segment (start 97 104.647387) (end 110.852613 118.5) (width 0.25) (layer "F.Cu") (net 7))
 (segment (start 108.89 83.49) (end 103.95 78.55) (width 0.25) (layer "F.Cu") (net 7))
 (segment (start 107.989009 115) (end 97.5 104.510991) (width 0.25) (layer "F.Cu") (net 13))
 (segment (start 97.5 104.510991) (end 97.5 79) (width 0.25) (layer "F.Cu") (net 13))
 (segment (start 101.86 79) (end 106.35 83.49) (width 0.25) (layer "F.Cu") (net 13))
 (segment (start 120 115) (end 107.989009 115) (width 0.25) (layer "F.Cu") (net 13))
 (segment (start 97.5 79) (end 101.86 79) (width 0.25) (layer "F.Cu") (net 13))
 (segment (start 120.08 111.5) (end 118.94863 111.5) (width 0.25) (layer "F.Cu") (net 1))
 (segment (start 118.94863 111.5) (end 107.715 100.26637) (width 0.25) (layer "F.Cu") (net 1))
 (segment (start 107.715 100.26637) (end 107.715 87.395) (width 0.25) (layer "F.Cu") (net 1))
 (segment (start 107.715 87.395) (end 103.81 83.49) (width 0.25) (layer "F.Cu") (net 1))
 (segment (start 137.08 125.92) (end 137.08 122.24) (width 0.25) (layer "F.Cu") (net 16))
 (segment (start 103 118.58) (end 103 125) (width 0.25) (layer "F.Cu") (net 16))
 (segment (start 136 127) (end 137.08 125.92) (width 0.25) (layer "F.Cu") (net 16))
 (segment (start 103 125) (end 105 127) (width 0.25) (layer "F.Cu") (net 16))
 (segment (start 105 127) (end 136 127) (width 0.25) (layer "F.Cu") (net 16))
 (segment (start 130.24 111.5) (end 134.54 107.2) (width 0.25) (layer "F.Cu") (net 2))
 (segment (start 134.54 107.2) (end 134.54 107) (width 0.25) (layer "F.Cu") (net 2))
 (segment (start 129.115 113.955) (end 129.115 109.885) (width 0.25) (layer "F.Cu") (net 10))
 (segment (start 129.115 109.885) (end 132 107) (width 0.25) (layer "F.Cu") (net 10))
 (segment (start 130.16 115) (end 129.115 113.955) (width 0.25) (layer "F.Cu") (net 10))
 (segment (start 124.38 112.72) (end 124.38 107) (width 0.25) (layer "B.Cu") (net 8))
 (segment (start 130.16 118.5) (end 124.38 112.72) (width 0.25) (layer "B.Cu") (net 8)))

